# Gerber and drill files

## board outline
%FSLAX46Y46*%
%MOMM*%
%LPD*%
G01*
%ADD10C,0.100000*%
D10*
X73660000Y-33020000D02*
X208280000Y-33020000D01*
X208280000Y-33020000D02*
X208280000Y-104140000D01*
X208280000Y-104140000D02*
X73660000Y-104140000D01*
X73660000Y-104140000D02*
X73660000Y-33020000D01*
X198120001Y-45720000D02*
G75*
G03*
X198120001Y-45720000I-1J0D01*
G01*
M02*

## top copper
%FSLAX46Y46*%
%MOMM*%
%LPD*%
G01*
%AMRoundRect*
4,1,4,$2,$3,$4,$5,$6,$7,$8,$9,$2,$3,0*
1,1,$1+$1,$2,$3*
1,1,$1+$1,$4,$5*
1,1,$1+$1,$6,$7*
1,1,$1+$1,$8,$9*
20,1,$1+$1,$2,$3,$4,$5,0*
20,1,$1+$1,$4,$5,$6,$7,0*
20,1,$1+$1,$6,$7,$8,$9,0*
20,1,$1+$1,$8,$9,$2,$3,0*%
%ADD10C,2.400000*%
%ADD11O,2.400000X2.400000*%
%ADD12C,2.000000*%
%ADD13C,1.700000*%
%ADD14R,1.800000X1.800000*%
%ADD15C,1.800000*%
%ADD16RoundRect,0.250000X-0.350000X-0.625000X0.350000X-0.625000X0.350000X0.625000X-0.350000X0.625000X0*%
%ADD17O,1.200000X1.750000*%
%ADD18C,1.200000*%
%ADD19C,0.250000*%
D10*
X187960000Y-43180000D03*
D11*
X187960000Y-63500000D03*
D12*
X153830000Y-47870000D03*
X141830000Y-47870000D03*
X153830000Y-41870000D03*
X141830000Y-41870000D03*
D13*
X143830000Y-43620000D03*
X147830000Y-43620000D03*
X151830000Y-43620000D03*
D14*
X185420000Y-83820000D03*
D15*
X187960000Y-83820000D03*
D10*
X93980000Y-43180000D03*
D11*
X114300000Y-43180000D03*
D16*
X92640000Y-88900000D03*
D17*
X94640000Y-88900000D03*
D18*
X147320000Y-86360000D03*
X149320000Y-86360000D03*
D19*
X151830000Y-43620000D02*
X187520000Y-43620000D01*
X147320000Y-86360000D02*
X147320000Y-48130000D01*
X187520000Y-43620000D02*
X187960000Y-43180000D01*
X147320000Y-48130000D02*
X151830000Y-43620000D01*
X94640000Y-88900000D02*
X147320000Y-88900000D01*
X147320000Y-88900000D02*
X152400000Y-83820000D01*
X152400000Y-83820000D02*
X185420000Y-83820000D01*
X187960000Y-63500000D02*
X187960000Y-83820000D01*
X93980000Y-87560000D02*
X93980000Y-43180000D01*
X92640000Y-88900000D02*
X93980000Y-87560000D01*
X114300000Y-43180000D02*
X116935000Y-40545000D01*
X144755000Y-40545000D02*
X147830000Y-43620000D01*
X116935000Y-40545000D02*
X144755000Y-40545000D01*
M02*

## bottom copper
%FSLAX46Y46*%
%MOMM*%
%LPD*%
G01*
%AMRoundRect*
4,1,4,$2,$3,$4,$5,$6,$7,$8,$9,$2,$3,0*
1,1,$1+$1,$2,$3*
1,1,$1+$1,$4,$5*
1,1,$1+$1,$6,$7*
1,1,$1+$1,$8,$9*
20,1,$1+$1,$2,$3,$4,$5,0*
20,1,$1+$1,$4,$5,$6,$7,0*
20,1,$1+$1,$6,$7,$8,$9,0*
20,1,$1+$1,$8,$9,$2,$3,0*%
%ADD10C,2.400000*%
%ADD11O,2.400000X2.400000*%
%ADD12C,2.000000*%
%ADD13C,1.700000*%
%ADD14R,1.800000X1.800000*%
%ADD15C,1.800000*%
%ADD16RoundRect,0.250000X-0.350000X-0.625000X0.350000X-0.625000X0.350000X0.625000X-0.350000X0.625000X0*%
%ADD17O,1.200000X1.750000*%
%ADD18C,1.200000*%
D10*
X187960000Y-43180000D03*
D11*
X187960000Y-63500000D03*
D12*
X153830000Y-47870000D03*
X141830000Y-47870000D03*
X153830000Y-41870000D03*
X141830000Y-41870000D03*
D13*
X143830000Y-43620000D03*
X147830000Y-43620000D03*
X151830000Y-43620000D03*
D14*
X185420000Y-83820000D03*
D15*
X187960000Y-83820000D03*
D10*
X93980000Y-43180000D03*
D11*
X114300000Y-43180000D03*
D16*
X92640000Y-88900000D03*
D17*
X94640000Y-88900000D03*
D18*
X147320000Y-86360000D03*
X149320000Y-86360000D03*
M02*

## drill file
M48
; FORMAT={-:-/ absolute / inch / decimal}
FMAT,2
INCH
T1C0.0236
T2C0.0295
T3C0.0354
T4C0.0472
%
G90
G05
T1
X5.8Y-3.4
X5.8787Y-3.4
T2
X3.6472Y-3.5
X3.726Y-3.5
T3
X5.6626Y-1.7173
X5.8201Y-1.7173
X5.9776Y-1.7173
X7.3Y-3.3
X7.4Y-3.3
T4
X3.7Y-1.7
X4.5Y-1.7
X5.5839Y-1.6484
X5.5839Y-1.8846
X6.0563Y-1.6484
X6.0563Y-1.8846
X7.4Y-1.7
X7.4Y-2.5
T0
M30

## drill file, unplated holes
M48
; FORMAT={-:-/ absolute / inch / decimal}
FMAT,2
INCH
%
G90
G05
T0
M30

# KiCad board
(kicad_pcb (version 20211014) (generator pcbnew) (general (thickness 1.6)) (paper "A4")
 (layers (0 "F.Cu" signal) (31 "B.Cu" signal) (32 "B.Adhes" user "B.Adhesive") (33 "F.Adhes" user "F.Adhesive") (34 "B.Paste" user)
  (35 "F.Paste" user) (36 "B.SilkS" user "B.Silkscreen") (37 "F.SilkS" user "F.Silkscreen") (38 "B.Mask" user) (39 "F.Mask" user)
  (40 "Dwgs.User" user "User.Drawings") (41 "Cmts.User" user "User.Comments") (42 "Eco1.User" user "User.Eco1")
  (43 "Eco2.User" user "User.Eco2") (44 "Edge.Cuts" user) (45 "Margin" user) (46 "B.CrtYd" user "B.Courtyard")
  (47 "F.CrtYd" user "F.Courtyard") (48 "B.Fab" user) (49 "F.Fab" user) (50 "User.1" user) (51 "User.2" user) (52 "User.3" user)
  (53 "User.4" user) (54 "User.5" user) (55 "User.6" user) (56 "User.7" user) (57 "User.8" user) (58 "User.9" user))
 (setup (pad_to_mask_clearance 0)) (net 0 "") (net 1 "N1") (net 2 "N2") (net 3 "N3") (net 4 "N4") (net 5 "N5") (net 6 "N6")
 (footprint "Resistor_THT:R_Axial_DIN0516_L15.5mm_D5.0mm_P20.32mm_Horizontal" (layer "F.Cu") (at 187.96 43.18 -90)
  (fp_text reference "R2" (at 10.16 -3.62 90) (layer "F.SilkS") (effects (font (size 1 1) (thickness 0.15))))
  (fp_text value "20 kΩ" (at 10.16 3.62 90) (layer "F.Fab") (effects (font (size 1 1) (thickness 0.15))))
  (pad "1" thru_hole circle (at 0 0 270) (size 2.4 2.4) (drill 1.2) (layers *.Cu *.Mask) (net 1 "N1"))
  (pad "2" thru_hole oval (at 20.32 0 270) (size 2.4 2.4) (drill 1.2) (layers *.Cu *.Mask) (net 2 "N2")))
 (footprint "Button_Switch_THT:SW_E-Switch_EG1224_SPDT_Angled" (layer "F.Cu") (at 143.83 43.62)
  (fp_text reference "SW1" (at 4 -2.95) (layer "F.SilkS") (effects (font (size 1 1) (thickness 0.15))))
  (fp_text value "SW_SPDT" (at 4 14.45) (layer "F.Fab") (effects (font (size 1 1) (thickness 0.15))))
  (pad "" thru_hole circle (at 10 4.25) (size 2 2) (drill 1.2) (layers *.Cu *.Mask))
  (pad "" thru_hole circle (at -2 4.25) (size 2 2) (drill 1.2) (layers *.Cu *.Mask))
  (pad "" thru_hole circle (at 10 -1.75) (size 2 2) (drill 1.2) (layers *.Cu *.Mask))
  (pad "" thru_hole circle (at -2 -1.75) (size 2 2) (drill 1.2) (layers *.Cu *.Mask))
  (pad "1" thru_hole circle (at 0 0) (size 1.7 1.7) (drill 0.9) (layers *.Cu *.Mask) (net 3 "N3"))
  (pad "2" thru_hole circle (at 4 0) (size 1.7 1.7) (drill 0.9) (layers *.Cu *.Mask) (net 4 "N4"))
  (pad "3" thru_hole circle (at 8 0) (size 1.7 1.7) (drill 0.9) (layers *.Cu *.Mask) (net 1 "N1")))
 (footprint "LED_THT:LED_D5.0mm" (layer "F.Cu") (at 185.42 83.82)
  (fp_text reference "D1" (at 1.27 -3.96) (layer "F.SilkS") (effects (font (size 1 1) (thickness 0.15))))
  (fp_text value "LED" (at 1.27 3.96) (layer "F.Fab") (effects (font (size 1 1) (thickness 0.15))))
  (pad "1" thru_hole rect (at 0 0) (size 1.8 1.8) (drill 0.9) (layers *.Cu *.Mask) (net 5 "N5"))
  (pad "2" thru_hole circle (at 2.54 0) (size 1.8 1.8) (drill 0.9) (layers *.Cu *.Mask) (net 2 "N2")))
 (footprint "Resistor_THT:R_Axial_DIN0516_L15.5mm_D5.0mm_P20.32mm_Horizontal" (layer "F.Cu") (at 93.98 43.18)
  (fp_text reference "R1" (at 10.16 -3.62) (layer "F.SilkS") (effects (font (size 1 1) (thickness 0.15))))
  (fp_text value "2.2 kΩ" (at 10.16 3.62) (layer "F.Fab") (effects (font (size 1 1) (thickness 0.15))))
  (pad "1" thru_hole circle (at 0 0) (size 2.4 2.4) (drill 1.2) (layers *.Cu *.Mask) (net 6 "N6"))
  (pad "2" thru_hole oval (at 20.32 0) (size 2.4 2.4) (drill 1.2) (layers *.Cu *.Mask) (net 4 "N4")))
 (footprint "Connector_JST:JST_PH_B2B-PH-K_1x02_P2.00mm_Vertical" (layer "F.Cu") (at 92.64 88.9)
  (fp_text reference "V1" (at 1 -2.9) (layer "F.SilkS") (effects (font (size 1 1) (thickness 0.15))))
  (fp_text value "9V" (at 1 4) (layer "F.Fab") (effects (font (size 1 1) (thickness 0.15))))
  (pad "1" thru_hole roundrect (at 0 0) (size 1.2 1.75) (drill 0.75) (layers *.Cu *.Mask) (roundrect_rratio 0.2083333333) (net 6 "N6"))
  (pad "2" thru_hole oval (at 2 0) (size 1.2 1.75) (drill 0.75) (layers *.Cu *.Mask) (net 5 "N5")))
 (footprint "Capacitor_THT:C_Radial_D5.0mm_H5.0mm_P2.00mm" (layer "F.Cu") (at 147.32 86.36)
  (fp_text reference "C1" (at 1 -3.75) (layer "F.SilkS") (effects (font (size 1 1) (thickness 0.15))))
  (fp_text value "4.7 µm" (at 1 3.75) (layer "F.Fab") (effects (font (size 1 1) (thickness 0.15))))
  (pad "1" thru_hole circle (at 0 0) (size 1.2 1.2) (drill 0.6) (layers *.Cu *.Mask) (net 1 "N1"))
  (pad "2" thru_hole circle (at 2 0) (size 1.2 1.2) (drill 0.6) (layers *.Cu *.Mask) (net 5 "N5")))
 (gr_rect (start 73.66 33.02) (end 208.28 104.14) (layer "Edge.Cuts") (width 0.1) (fill none))
 (gr_circle (center 198.12 45.72) (end 198.12 45.72) (layer "Edge.Cuts") (width 0.1) (fill none))
 (segment (start 151.83 43.62) (end 187.52 43.62) (width 0.25) (layer "F.Cu") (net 1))
 (segment (start 147.32 86.36) (end 147.32 48.13) (width 0.25) (layer "F.Cu") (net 1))
 (segment (start 187.52 43.62) (end 187.96 43.18) (width 0.25) (layer "F.Cu") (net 1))
 (segment (start 147.32 48.13) (end 151.83 43.62) (width 0.25) (layer "F.Cu") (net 1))
 (segment (start 94.64 88.9) (end 147.32 88.9) (width 0.25) (layer "F.Cu") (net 5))
 (segment (start 147.32 88.9) (end 152.4 83.82) (width 0.25) (layer "F.Cu") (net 5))
 (segment (start 152.4 83.82) (end 185.42 83.82) (width 0.25) (layer "F.Cu") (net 5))
 (segment (start 187.96 63.5) (end 187.96 83.82) (width 0.25) (layer "F.Cu") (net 2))
 (segment (start 93.98 87.56) (end 93.98 43.18) (width 0.25) (layer "F.Cu") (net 6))
 (segment (start 92.64 88.9) (end 93.98 87.56) (width 0.25) (layer "F.Cu") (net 6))
 (segment (start 114.3 43.18) (end 116.935 40.545) (width 0.25) (layer "F.Cu") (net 4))
 (segment (start 144.755 40.545) (end 147.83 43.62) (width 0.25) (layer "F.Cu") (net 4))
 (segment (start 116.935 40.545) (end 144.755 40.545) (width 0.25) (layer "F.Cu") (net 4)))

